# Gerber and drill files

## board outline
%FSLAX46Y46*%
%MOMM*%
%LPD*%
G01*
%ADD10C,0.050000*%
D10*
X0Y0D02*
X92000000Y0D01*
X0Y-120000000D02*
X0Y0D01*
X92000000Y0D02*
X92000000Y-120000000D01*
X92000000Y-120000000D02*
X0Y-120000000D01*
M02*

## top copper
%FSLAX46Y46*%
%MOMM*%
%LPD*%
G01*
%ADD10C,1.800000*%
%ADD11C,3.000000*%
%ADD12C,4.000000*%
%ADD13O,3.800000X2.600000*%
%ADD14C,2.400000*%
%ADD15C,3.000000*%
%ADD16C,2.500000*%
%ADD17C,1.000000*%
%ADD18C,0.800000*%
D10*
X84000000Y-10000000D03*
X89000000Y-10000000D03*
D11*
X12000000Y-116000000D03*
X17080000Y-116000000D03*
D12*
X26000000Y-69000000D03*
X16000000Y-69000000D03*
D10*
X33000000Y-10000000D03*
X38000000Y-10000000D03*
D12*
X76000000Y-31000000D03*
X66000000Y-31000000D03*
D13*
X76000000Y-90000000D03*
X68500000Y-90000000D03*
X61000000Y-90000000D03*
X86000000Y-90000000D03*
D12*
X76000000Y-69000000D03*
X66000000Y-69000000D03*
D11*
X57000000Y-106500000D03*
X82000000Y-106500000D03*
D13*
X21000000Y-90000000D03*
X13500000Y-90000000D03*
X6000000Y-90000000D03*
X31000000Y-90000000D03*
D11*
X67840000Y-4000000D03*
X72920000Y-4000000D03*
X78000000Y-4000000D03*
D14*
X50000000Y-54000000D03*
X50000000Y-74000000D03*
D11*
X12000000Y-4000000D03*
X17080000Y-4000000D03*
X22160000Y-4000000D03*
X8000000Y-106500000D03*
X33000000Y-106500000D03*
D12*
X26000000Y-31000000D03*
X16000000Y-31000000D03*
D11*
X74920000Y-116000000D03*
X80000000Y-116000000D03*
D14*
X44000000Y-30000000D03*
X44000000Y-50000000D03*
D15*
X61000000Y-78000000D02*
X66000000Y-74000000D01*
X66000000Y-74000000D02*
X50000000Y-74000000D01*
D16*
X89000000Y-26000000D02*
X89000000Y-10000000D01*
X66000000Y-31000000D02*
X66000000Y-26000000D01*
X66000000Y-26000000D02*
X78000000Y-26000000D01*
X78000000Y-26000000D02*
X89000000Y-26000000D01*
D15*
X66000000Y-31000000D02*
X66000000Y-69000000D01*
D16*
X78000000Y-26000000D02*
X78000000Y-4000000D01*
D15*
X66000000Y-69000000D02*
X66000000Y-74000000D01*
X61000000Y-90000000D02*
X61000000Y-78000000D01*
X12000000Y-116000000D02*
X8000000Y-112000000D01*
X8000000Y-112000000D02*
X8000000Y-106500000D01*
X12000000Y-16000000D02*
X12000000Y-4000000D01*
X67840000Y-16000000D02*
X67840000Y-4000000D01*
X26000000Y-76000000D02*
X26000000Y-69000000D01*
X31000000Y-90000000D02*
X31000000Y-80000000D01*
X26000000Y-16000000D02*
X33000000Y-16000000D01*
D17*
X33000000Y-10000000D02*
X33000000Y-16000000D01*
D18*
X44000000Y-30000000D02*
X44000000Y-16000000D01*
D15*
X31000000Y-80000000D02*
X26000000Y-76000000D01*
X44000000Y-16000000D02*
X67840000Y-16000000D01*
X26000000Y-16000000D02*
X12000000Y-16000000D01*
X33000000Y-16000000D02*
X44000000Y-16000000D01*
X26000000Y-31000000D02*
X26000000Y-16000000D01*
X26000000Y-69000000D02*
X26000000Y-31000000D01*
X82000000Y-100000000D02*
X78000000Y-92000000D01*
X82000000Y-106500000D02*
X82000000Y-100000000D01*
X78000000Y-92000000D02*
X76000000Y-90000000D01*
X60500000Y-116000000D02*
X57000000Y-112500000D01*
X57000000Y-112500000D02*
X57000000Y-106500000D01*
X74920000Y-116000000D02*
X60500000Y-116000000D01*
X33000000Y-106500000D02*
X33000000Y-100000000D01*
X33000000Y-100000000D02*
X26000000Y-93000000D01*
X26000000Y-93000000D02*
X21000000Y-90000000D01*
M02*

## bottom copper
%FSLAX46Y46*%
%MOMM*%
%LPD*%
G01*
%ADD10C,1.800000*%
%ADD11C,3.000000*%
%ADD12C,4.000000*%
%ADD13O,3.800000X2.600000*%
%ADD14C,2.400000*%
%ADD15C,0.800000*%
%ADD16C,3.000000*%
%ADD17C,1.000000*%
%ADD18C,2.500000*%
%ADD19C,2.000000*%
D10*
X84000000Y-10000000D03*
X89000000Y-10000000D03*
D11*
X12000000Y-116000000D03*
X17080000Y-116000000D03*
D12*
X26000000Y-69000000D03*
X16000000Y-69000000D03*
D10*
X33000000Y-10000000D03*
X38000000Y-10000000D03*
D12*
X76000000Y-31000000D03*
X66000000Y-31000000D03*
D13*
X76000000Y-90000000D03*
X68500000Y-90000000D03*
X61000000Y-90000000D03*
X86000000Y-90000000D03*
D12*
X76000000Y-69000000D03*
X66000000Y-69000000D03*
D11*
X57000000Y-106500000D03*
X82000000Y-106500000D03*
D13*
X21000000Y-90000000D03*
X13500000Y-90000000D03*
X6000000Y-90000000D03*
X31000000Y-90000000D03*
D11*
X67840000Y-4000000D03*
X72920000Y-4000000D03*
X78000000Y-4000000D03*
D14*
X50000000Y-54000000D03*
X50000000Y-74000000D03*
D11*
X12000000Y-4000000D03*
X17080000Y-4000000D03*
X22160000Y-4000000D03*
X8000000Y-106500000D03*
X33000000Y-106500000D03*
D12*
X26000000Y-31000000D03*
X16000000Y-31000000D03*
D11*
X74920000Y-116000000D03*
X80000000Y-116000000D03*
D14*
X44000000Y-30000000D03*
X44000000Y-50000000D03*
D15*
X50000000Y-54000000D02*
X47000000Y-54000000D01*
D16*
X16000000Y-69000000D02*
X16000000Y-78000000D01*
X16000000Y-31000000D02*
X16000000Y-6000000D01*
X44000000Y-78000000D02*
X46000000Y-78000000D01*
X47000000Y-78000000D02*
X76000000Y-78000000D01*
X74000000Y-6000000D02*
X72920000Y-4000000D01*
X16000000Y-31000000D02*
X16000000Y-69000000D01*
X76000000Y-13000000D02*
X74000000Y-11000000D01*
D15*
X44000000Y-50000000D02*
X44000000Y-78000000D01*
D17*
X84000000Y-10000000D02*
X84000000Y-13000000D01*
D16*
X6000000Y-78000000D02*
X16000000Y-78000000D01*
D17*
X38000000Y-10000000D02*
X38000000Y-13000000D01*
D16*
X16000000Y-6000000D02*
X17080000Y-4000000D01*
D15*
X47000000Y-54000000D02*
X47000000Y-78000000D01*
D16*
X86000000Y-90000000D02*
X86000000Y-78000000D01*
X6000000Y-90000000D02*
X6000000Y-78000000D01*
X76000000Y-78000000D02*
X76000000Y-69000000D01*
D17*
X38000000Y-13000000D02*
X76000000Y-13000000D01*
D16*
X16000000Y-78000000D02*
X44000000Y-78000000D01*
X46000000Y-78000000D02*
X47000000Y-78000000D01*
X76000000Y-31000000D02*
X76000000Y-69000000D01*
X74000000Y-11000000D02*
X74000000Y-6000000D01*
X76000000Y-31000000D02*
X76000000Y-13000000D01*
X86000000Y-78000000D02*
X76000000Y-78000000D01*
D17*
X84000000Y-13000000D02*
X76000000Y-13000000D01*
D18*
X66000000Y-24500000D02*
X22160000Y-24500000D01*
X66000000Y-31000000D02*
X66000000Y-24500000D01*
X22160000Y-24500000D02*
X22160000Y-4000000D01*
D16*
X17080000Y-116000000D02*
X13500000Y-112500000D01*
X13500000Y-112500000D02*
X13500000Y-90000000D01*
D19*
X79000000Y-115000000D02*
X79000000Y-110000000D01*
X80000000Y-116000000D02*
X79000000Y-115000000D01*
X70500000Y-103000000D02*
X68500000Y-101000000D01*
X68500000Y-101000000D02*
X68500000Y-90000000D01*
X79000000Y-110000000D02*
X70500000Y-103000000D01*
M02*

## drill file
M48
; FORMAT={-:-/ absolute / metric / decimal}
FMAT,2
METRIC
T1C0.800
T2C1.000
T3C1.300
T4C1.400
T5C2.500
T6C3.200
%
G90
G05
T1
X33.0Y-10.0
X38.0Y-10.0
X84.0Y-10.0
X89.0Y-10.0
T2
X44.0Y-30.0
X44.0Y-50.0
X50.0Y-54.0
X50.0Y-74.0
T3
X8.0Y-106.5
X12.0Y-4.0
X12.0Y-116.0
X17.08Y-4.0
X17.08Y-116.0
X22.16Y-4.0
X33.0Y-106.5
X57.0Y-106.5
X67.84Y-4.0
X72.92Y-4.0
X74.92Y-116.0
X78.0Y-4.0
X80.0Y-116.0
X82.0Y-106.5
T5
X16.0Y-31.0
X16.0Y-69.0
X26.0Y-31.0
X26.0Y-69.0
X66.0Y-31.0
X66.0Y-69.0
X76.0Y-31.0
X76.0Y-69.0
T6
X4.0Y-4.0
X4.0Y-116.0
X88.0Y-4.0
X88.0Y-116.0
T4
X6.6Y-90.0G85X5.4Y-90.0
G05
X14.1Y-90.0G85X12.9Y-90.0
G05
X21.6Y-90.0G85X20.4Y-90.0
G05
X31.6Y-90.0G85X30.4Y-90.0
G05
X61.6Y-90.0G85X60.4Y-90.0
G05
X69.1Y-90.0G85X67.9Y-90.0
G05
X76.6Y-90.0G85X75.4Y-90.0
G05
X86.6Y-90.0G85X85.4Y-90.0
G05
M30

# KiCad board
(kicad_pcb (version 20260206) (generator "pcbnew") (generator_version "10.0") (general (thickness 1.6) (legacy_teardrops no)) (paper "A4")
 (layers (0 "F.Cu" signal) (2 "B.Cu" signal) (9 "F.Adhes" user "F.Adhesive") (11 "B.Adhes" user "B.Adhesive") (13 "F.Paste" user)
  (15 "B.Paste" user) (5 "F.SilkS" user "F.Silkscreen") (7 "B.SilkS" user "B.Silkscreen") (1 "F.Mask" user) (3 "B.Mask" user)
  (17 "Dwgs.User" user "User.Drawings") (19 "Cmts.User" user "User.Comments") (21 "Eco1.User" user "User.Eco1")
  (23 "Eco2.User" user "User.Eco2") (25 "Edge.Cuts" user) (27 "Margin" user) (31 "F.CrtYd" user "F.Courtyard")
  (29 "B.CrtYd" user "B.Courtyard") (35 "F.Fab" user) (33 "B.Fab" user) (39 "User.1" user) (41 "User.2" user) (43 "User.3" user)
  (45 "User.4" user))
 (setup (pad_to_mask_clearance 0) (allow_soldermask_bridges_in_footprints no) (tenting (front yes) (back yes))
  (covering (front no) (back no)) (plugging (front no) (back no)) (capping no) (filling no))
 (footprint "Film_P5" (layer "F.Cu") (at 84 10)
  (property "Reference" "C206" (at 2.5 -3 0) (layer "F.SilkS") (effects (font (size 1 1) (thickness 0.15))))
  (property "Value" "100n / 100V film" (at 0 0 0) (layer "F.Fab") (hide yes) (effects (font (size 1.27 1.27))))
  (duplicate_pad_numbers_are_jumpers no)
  (pad "1" thru_hole circle (at 0 0) (size 1.8 1.8) (drill 0.8) (layers "*.Cu" "*.Mask") (remove_unused_layers no) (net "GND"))
  (pad "2" thru_hole circle (at 5 0) (size 1.8 1.8) (drill 0.8) (layers "*.Cu" "*.Mask") (remove_unused_layers no) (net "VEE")))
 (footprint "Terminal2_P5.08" (layer "F.Cu") (at 12 116)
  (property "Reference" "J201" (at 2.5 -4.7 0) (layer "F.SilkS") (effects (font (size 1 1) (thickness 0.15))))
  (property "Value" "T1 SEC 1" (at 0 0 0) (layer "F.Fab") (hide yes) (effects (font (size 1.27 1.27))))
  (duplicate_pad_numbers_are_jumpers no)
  (pad "1" thru_hole circle (at 0 0) (size 3 3) (drill 1.3) (layers "*.Cu" "*.Mask") (remove_unused_layers no) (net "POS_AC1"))
  (pad "2" thru_hole circle (at 5.08 0) (size 3 3) (drill 1.3) (layers "*.Cu" "*.Mask") (remove_unused_layers no) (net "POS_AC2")))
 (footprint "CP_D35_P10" (layer "F.Cu") (at 26 69 180)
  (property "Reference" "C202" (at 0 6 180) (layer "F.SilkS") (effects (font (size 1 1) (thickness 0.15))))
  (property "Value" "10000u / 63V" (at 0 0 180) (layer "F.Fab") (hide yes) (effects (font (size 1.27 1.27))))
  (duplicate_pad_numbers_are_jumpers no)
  (pad "1" thru_hole circle (at 0 0 180) (size 4 4) (drill 2.5) (layers "*.Cu" "*.Mask") (remove_unused_layers no) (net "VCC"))
  (pad "2" thru_hole circle (at 10 0 180) (size 4 4) (drill 2.5) (layers "*.Cu" "*.Mask") (remove_unused_layers no) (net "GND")))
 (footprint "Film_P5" (layer "F.Cu") (at 33 10)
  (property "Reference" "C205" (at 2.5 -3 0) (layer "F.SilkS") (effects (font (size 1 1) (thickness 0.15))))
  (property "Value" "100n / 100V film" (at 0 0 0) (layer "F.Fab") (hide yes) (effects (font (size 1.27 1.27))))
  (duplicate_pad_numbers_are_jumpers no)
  (pad "1" thru_hole circle (at 0 0) (size 1.8 1.8) (drill 0.8) (layers "*.Cu" "*.Mask") (remove_unused_layers no) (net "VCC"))
  (pad "2" thru_hole circle (at 5 0) (size 1.8 1.8) (drill 0.8) (layers "*.Cu" "*.Mask") (remove_unused_layers no) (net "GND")))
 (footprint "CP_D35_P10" (layer "F.Cu") (at 76 31 180)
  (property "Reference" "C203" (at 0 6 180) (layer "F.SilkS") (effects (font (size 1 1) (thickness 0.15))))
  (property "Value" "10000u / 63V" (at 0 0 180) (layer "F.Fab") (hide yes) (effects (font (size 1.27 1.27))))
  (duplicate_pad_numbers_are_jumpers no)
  (pad "1" thru_hole circle (at 0 0 180) (size 4 4) (drill 2.5) (layers "*.Cu" "*.Mask") (remove_unused_layers no) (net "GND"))
  (pad "2" thru_hole circle (at 10 0 180) (size 4 4) (drill 2.5) (layers "*.Cu" "*.Mask") (remove_unused_layers no) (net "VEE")))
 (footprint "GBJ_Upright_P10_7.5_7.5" (layer "F.Cu") (at 86 90 180)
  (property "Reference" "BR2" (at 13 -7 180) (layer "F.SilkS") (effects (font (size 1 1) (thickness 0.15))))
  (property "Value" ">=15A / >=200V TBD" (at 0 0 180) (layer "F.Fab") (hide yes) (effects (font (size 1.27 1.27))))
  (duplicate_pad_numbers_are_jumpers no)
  (pad "AC1" thru_hole oval (at 10 0 180) (size 3.8 2.6) (drill oval 2.6 1.4) (layers "*.Cu" "*.Mask") (remove_unused_layers no)
   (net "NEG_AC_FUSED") (thermal_bridge_angle 45))
  (pad "AC2" thru_hole oval (at 17.5 0 180) (size 3.8 2.6) (drill oval 2.6 1.4) (layers "*.Cu" "*.Mask") (remove_unused_layers no)
   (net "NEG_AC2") (thermal_bridge_angle 45))
  (pad "N" thru_hole oval (at 25 0 180) (size 3.8 2.6) (drill oval 2.6 1.4) (layers "*.Cu" "*.Mask") (remove_unused_layers no) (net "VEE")
   (thermal_bridge_angle 45))
  (pad "P" thru_hole oval (at 0 0 180) (size 3.8 2.6) (drill oval 2.6 1.4) (layers "*.Cu" "*.Mask") (remove_unused_layers no) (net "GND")
   (thermal_bridge_angle 45)))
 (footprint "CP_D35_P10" (layer "F.Cu") (at 76 69 180)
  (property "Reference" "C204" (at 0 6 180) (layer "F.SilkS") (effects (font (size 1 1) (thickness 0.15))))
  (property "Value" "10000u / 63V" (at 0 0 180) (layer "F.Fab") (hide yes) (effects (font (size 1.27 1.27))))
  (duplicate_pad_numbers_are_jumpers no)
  (pad "1" thru_hole circle (at 0 0 180) (size 4 4) (drill 2.5) (layers "*.Cu" "*.Mask") (remove_unused_layers no) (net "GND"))
  (pad "2" thru_hole circle (at 10 0 180) (size 4 4) (drill 2.5) (layers "*.Cu" "*.Mask") (remove_unused_layers no) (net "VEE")))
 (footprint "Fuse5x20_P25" (layer "F.Cu") (at 57 106.5)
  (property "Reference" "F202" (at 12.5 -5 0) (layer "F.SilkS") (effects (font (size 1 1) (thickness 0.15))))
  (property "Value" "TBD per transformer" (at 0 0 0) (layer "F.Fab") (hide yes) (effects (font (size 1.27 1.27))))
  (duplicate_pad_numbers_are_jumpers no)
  (pad "1" thru_hole circle (at 0 0) (size 3 3) (drill 1.3) (layers "*.Cu" "*.Mask") (remove_unused_layers no) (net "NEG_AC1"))
  (pad "2" thru_hole circle (at 25 0) (size 3 3) (drill 1.3) (layers "*.Cu" "*.Mask") (remove_unused_layers no) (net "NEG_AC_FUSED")))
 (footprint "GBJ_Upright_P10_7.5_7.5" (layer "F.Cu") (at 31 90 180)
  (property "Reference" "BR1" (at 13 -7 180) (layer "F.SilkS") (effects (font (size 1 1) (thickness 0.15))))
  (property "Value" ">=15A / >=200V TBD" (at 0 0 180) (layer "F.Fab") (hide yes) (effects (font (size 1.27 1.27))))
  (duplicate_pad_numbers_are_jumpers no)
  (pad "AC1" thru_hole oval (at 10 0 180) (size 3.8 2.6) (drill oval 2.6 1.4) (layers "*.Cu" "*.Mask") (remove_unused_layers no)
   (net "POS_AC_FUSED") (thermal_bridge_angle 45))
  (pad "AC2" thru_hole oval (at 17.5 0 180) (size 3.8 2.6) (drill oval 2.6 1.4) (layers "*.Cu" "*.Mask") (remove_unused_layers no)
   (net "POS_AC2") (thermal_bridge_angle 45))
  (pad "N" thru_hole oval (at 25 0 180) (size 3.8 2.6) (drill oval 2.6 1.4) (layers "*.Cu" "*.Mask") (remove_unused_layers no) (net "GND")
   (thermal_bridge_angle 45))
  (pad "P" thru_hole oval (at 0 0 180) (size 3.8 2.6) (drill oval 2.6 1.4) (layers "*.Cu" "*.Mask") (remove_unused_layers no) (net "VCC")
   (thermal_bridge_angle 45)))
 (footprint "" (layer "F.Cu") (at 88 4)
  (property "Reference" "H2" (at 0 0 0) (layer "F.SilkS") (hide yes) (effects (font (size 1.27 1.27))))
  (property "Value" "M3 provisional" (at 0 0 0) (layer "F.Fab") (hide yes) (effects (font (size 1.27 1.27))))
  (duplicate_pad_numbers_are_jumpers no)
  (pad "" np_thru_hole circle (at 0 0) (size 3.2 3.2) (drill 3.2) (layers "*.Cu" "*.Mask")))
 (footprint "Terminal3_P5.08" (layer "F.Cu") (at 67.84 4)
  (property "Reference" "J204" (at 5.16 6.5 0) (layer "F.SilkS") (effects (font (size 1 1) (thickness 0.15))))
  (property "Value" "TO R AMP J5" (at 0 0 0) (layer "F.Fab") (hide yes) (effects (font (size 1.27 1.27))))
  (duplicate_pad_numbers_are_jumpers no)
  (pad "1" thru_hole circle (at 0 0) (size 3 3) (drill 1.3) (layers "*.Cu" "*.Mask") (remove_unused_layers no) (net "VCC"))
  (pad "2" thru_hole circle (at 5.08 0) (size 3 3) (drill 1.3) (layers "*.Cu" "*.Mask") (remove_unused_layers no) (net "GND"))
  (pad "3" thru_hole circle (at 10.16 0) (size 3 3) (drill 1.3) (layers "*.Cu" "*.Mask") (remove_unused_layers no) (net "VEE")))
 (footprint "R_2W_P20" (layer "F.Cu") (at 50 54 -90)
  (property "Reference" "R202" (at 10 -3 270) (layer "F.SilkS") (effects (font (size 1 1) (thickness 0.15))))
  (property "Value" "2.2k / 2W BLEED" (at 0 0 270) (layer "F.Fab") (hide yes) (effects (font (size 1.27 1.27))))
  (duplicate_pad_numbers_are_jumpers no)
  (pad "1" thru_hole circle (at 0 0 270) (size 2.4 2.4) (drill 1) (layers "*.Cu" "*.Mask") (remove_unused_layers no) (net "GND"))
  (pad "2" thru_hole circle (at 20 0 270) (size 2.4 2.4) (drill 1) (layers "*.Cu" "*.Mask") (remove_unused_layers no) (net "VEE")))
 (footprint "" (layer "F.Cu") (at 4 4)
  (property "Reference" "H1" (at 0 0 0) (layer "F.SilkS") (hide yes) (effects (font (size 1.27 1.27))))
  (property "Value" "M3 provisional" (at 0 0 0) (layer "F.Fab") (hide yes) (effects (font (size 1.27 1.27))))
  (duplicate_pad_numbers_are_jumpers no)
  (pad "" np_thru_hole circle (at 0 0) (size 3.2 3.2) (drill 3.2) (layers "*.Cu" "*.Mask")))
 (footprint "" (layer "F.Cu") (at 4 116)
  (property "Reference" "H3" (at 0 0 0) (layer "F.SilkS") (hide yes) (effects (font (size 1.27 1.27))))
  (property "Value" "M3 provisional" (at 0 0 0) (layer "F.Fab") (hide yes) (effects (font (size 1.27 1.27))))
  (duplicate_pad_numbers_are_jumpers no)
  (pad "" np_thru_hole circle (at 0 0) (size 3.2 3.2) (drill 3.2) (layers "*.Cu" "*.Mask")))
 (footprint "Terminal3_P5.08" (layer "F.Cu") (at 12 4)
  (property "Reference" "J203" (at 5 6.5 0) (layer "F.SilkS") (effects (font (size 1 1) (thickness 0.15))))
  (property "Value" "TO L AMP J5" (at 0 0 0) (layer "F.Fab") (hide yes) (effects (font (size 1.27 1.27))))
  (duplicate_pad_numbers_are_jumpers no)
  (pad "1" thru_hole circle (at 0 0) (size 3 3) (drill 1.3) (layers "*.Cu" "*.Mask") (remove_unused_layers no) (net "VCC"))
  (pad "2" thru_hole circle (at 5.08 0) (size 3 3) (drill 1.3) (layers "*.Cu" "*.Mask") (remove_unused_layers no) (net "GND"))
  (pad "3" thru_hole circle (at 10.16 0) (size 3 3) (drill 1.3) (layers "*.Cu" "*.Mask") (remove_unused_layers no) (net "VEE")))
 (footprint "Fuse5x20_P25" (layer "F.Cu") (at 8 106.5)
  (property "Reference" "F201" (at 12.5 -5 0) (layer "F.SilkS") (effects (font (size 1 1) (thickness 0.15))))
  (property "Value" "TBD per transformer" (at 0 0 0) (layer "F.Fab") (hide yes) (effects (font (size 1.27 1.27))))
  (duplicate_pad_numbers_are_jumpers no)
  (pad "1" thru_hole circle (at 0 0) (size 3 3) (drill 1.3) (layers "*.Cu" "*.Mask") (remove_unused_layers no) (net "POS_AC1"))
  (pad "2" thru_hole circle (at 25 0) (size 3 3) (drill 1.3) (layers "*.Cu" "*.Mask") (remove_unused_layers no) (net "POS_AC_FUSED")))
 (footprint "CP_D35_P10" (layer "F.Cu") (at 26 31 180)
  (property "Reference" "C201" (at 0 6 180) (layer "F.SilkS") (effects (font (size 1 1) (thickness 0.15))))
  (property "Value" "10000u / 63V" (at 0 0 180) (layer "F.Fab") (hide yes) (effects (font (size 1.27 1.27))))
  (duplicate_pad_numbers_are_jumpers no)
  (pad "1" thru_hole circle (at 0 0 180) (size 4 4) (drill 2.5) (layers "*.Cu" "*.Mask") (remove_unused_layers no) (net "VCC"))
  (pad "2" thru_hole circle (at 10 0 180) (size 4 4) (drill 2.5) (layers "*.Cu" "*.Mask") (remove_unused_layers no) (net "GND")))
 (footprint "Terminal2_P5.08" (layer "F.Cu") (at 74.92 116)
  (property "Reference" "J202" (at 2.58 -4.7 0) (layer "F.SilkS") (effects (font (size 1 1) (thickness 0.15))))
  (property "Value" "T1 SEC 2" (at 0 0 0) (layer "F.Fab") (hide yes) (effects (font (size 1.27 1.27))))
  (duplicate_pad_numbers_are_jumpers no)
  (pad "1" thru_hole circle (at 0 0) (size 3 3) (drill 1.3) (layers "*.Cu" "*.Mask") (remove_unused_layers no) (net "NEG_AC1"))
  (pad "2" thru_hole circle (at 5.08 0) (size 3 3) (drill 1.3) (layers "*.Cu" "*.Mask") (remove_unused_layers no) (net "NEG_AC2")))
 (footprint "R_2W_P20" (layer "F.Cu") (at 44 30 -90)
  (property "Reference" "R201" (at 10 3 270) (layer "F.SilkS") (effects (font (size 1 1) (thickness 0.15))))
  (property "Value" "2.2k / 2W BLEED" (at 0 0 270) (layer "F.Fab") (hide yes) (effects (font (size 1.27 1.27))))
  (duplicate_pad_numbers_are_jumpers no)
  (pad "1" thru_hole circle (at 0 0 270) (size 2.4 2.4) (drill 1) (layers "*.Cu" "*.Mask") (remove_unused_layers no) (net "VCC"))
  (pad "2" thru_hole circle (at 20 0 270) (size 2.4 2.4) (drill 1) (layers "*.Cu" "*.Mask") (remove_unused_layers no) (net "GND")))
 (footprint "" (layer "F.Cu") (at 88 116)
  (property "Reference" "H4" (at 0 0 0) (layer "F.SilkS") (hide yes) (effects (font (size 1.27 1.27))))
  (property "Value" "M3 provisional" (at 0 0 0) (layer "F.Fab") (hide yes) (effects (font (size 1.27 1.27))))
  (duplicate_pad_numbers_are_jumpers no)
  (pad "" np_thru_hole circle (at 0 0) (size 3.2 3.2) (drill 3.2) (layers "*.Cu" "*.Mask")))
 (gr_line (start 0 0) (end 92 0) (stroke (width 0.05) (type default)) (layer "Edge.Cuts"))
 (gr_line (start 0 120) (end 0 0) (stroke (width 0.05) (type default)) (layer "Edge.Cuts"))
 (gr_line (start 92 0) (end 92 120) (stroke (width 0.05) (type default)) (layer "Edge.Cuts"))
 (gr_line (start 92 120) (end 0 120) (stroke (width 0.05) (type default)) (layer "Edge.Cuts"))
 (segment (start 50 54) (end 47 54) (width 0.8) (layer "B.Cu") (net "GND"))
 (segment (start 16 69) (end 16 78) (width 3) (layer "B.Cu") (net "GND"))
 (segment (start 16 31) (end 16 6) (width 3) (layer "B.Cu") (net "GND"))
 (segment (start 44 78) (end 46 78) (width 3) (layer "B.Cu") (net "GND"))
 (segment (start 47 78) (end 76 78) (width 3) (layer "B.Cu") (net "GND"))
 (segment (start 74 6) (end 72.92 4) (width 3) (layer "B.Cu") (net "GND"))
 (segment (start 16 31) (end 16 69) (width 3) (layer "B.Cu") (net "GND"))
 (segment (start 76 13) (end 74 11) (width 3) (layer "B.Cu") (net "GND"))
 (segment (start 44 50) (end 44 78) (width 0.8) (layer "B.Cu") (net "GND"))
 (segment (start 84 10) (end 84 13) (width 1) (layer "B.Cu") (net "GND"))
 (segment (start 6 78) (end 16 78) (width 3) (layer "B.Cu") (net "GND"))
 (segment (start 38 10) (end 38 13) (width 1) (layer "B.Cu") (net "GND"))
 (segment (start 16 6) (end 17.08 4) (width 3) (layer "B.Cu") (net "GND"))
 (segment (start 47 54) (end 47 78) (width 0.8) (layer "B.Cu") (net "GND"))
 (segment (start 86 90) (end 86 78) (width 3) (layer "B.Cu") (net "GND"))
 (segment (start 6 90) (end 6 78) (width 3) (layer "B.Cu") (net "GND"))
 (segment (start 76 78) (end 76 69) (width 3) (layer "B.Cu") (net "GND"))
 (segment (start 38 13) (end 76 13) (width 1) (layer "B.Cu") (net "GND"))
 (segment (start 16 78) (end 44 78) (width 3) (layer "B.Cu") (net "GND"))
 (segment (start 46 78) (end 47 78) (width 3) (layer "B.Cu") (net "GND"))
 (segment (start 76 31) (end 76 69) (width 3) (layer "B.Cu") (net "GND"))
 (segment (start 74 11) (end 74 6) (width 3) (layer "B.Cu") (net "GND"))
 (segment (start 76 31) (end 76 13) (width 3) (layer "B.Cu") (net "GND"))
 (segment (start 86 78) (end 76 78) (width 3) (layer "B.Cu") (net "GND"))
 (segment (start 84 13) (end 76 13) (width 1) (layer "B.Cu") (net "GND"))
 (segment (start 61 78) (end 66 74) (width 3) (layer "F.Cu") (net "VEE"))
 (segment (start 66 74) (end 50 74) (width 3) (layer "F.Cu") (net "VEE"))
 (segment (start 89 26) (end 89 10) (width 2.5) (layer "F.Cu") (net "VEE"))
 (segment (start 66 31) (end 66 26) (width 2.5) (layer "F.Cu") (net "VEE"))
 (segment (start 66 26) (end 78 26) (width 2.5) (layer "F.Cu") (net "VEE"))
 (segment (start 78 26) (end 89 26) (width 2.5) (layer "F.Cu") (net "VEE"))
 (segment (start 66 31) (end 66 69) (width 3) (layer "F.Cu") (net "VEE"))
 (segment (start 78 26) (end 78 4) (width 2.5) (layer "F.Cu") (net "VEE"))
 (segment (start 66 69) (end 66 74) (width 3) (layer "F.Cu") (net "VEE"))
 (segment (start 61 90) (end 61 78) (width 3) (layer "F.Cu") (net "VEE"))
 (segment (start 66 24.5) (end 22.16 24.5) (width 2.5) (layer "B.Cu") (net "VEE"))
 (segment (start 66 31) (end 66 24.5) (width 2.5) (layer "B.Cu") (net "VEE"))
 (segment (start 22.16 24.5) (end 22.16 4) (width 2.5) (layer "B.Cu") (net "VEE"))
 (segment (start 12 116) (end 8 112) (width 3) (layer "F.Cu") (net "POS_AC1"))
 (segment (start 8 112) (end 8 106.5) (width 3) (layer "F.Cu") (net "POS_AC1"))
 (segment (start 17.08 116) (end 13.5 112.5) (width 3) (layer "B.Cu") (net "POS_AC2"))
 (segment (start 13.5 112.5) (end 13.5 90) (width 3) (layer "B.Cu") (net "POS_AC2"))
 (segment (start 12 16) (end 12 4) (width 3) (layer "F.Cu") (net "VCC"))
 (segment (start 67.84 16) (end 67.84 4) (width 3) (layer "F.Cu") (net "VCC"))
 (segment (start 26 76) (end 26 69) (width 3) (layer "F.Cu") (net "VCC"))
 (segment (start 31 90) (end 31 80) (width 3) (layer "F.Cu") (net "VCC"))
 (segment (start 26 16) (end 33 16) (width 3) (layer "F.Cu") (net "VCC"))
 (segment (start 33 10) (end 33 16) (width 1) (layer "F.Cu") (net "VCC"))
 (segment (start 44 30) (end 44 16) (width 0.8) (layer "F.Cu") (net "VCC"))
 (segment (start 31 80) (end 26 76) (width 3) (layer "F.Cu") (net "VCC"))
 (segment (start 44 16) (end 67.84 16) (width 3) (layer "F.Cu") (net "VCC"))
 (segment (start 26 16) (end 12 16) (width 3) (layer "F.Cu") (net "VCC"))
 (segment (start 33 16) (end 44 16) (width 3) (layer "F.Cu") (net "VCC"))
 (segment (start 26 31) (end 26 16) (width 3) (layer "F.Cu") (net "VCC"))
 (segment (start 26 69) (end 26 31) (width 3) (layer "F.Cu") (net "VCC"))
 (segment (start 82 100) (end 78 92) (width 3) (layer "F.Cu") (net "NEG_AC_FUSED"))
 (segment (start 82 106.5) (end 82 100) (width 3) (layer "F.Cu") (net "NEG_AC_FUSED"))
 (segment (start 78 92) (end 76 90) (width 3) (layer "F.Cu") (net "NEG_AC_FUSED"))
 (segment (start 79 115) (end 79 110) (width 2) (layer "B.Cu") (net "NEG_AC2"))
 (segment (start 80 116) (end 79 115) (width 2) (layer "B.Cu") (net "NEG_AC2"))
 (segment (start 70.5 103) (end 68.5 101) (width 2) (layer "B.Cu") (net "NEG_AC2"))
 (segment (start 68.5 101) (end 68.5 90) (width 2) (layer "B.Cu") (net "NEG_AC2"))
 (segment (start 79 110) (end 70.5 103) (width 2) (layer "B.Cu") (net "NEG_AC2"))
 (segment (start 60.5 116) (end 57 112.5) (width 3) (layer "F.Cu") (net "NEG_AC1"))
 (segment (start 57 112.5) (end 57 106.5) (width 3) (layer "F.Cu") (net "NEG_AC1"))
 (segment (start 74.92 116) (end 60.5 116) (width 3) (layer "F.Cu") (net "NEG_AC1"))
 (segment (start 33 106.5) (end 33 100) (width 3) (layer "F.Cu") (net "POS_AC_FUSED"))
 (segment (start 33 100) (end 26 93) (width 3) (layer "F.Cu") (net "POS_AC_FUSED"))
 (segment (start 26 93) (end 21 90) (width 3) (layer "F.Cu") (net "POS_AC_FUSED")))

